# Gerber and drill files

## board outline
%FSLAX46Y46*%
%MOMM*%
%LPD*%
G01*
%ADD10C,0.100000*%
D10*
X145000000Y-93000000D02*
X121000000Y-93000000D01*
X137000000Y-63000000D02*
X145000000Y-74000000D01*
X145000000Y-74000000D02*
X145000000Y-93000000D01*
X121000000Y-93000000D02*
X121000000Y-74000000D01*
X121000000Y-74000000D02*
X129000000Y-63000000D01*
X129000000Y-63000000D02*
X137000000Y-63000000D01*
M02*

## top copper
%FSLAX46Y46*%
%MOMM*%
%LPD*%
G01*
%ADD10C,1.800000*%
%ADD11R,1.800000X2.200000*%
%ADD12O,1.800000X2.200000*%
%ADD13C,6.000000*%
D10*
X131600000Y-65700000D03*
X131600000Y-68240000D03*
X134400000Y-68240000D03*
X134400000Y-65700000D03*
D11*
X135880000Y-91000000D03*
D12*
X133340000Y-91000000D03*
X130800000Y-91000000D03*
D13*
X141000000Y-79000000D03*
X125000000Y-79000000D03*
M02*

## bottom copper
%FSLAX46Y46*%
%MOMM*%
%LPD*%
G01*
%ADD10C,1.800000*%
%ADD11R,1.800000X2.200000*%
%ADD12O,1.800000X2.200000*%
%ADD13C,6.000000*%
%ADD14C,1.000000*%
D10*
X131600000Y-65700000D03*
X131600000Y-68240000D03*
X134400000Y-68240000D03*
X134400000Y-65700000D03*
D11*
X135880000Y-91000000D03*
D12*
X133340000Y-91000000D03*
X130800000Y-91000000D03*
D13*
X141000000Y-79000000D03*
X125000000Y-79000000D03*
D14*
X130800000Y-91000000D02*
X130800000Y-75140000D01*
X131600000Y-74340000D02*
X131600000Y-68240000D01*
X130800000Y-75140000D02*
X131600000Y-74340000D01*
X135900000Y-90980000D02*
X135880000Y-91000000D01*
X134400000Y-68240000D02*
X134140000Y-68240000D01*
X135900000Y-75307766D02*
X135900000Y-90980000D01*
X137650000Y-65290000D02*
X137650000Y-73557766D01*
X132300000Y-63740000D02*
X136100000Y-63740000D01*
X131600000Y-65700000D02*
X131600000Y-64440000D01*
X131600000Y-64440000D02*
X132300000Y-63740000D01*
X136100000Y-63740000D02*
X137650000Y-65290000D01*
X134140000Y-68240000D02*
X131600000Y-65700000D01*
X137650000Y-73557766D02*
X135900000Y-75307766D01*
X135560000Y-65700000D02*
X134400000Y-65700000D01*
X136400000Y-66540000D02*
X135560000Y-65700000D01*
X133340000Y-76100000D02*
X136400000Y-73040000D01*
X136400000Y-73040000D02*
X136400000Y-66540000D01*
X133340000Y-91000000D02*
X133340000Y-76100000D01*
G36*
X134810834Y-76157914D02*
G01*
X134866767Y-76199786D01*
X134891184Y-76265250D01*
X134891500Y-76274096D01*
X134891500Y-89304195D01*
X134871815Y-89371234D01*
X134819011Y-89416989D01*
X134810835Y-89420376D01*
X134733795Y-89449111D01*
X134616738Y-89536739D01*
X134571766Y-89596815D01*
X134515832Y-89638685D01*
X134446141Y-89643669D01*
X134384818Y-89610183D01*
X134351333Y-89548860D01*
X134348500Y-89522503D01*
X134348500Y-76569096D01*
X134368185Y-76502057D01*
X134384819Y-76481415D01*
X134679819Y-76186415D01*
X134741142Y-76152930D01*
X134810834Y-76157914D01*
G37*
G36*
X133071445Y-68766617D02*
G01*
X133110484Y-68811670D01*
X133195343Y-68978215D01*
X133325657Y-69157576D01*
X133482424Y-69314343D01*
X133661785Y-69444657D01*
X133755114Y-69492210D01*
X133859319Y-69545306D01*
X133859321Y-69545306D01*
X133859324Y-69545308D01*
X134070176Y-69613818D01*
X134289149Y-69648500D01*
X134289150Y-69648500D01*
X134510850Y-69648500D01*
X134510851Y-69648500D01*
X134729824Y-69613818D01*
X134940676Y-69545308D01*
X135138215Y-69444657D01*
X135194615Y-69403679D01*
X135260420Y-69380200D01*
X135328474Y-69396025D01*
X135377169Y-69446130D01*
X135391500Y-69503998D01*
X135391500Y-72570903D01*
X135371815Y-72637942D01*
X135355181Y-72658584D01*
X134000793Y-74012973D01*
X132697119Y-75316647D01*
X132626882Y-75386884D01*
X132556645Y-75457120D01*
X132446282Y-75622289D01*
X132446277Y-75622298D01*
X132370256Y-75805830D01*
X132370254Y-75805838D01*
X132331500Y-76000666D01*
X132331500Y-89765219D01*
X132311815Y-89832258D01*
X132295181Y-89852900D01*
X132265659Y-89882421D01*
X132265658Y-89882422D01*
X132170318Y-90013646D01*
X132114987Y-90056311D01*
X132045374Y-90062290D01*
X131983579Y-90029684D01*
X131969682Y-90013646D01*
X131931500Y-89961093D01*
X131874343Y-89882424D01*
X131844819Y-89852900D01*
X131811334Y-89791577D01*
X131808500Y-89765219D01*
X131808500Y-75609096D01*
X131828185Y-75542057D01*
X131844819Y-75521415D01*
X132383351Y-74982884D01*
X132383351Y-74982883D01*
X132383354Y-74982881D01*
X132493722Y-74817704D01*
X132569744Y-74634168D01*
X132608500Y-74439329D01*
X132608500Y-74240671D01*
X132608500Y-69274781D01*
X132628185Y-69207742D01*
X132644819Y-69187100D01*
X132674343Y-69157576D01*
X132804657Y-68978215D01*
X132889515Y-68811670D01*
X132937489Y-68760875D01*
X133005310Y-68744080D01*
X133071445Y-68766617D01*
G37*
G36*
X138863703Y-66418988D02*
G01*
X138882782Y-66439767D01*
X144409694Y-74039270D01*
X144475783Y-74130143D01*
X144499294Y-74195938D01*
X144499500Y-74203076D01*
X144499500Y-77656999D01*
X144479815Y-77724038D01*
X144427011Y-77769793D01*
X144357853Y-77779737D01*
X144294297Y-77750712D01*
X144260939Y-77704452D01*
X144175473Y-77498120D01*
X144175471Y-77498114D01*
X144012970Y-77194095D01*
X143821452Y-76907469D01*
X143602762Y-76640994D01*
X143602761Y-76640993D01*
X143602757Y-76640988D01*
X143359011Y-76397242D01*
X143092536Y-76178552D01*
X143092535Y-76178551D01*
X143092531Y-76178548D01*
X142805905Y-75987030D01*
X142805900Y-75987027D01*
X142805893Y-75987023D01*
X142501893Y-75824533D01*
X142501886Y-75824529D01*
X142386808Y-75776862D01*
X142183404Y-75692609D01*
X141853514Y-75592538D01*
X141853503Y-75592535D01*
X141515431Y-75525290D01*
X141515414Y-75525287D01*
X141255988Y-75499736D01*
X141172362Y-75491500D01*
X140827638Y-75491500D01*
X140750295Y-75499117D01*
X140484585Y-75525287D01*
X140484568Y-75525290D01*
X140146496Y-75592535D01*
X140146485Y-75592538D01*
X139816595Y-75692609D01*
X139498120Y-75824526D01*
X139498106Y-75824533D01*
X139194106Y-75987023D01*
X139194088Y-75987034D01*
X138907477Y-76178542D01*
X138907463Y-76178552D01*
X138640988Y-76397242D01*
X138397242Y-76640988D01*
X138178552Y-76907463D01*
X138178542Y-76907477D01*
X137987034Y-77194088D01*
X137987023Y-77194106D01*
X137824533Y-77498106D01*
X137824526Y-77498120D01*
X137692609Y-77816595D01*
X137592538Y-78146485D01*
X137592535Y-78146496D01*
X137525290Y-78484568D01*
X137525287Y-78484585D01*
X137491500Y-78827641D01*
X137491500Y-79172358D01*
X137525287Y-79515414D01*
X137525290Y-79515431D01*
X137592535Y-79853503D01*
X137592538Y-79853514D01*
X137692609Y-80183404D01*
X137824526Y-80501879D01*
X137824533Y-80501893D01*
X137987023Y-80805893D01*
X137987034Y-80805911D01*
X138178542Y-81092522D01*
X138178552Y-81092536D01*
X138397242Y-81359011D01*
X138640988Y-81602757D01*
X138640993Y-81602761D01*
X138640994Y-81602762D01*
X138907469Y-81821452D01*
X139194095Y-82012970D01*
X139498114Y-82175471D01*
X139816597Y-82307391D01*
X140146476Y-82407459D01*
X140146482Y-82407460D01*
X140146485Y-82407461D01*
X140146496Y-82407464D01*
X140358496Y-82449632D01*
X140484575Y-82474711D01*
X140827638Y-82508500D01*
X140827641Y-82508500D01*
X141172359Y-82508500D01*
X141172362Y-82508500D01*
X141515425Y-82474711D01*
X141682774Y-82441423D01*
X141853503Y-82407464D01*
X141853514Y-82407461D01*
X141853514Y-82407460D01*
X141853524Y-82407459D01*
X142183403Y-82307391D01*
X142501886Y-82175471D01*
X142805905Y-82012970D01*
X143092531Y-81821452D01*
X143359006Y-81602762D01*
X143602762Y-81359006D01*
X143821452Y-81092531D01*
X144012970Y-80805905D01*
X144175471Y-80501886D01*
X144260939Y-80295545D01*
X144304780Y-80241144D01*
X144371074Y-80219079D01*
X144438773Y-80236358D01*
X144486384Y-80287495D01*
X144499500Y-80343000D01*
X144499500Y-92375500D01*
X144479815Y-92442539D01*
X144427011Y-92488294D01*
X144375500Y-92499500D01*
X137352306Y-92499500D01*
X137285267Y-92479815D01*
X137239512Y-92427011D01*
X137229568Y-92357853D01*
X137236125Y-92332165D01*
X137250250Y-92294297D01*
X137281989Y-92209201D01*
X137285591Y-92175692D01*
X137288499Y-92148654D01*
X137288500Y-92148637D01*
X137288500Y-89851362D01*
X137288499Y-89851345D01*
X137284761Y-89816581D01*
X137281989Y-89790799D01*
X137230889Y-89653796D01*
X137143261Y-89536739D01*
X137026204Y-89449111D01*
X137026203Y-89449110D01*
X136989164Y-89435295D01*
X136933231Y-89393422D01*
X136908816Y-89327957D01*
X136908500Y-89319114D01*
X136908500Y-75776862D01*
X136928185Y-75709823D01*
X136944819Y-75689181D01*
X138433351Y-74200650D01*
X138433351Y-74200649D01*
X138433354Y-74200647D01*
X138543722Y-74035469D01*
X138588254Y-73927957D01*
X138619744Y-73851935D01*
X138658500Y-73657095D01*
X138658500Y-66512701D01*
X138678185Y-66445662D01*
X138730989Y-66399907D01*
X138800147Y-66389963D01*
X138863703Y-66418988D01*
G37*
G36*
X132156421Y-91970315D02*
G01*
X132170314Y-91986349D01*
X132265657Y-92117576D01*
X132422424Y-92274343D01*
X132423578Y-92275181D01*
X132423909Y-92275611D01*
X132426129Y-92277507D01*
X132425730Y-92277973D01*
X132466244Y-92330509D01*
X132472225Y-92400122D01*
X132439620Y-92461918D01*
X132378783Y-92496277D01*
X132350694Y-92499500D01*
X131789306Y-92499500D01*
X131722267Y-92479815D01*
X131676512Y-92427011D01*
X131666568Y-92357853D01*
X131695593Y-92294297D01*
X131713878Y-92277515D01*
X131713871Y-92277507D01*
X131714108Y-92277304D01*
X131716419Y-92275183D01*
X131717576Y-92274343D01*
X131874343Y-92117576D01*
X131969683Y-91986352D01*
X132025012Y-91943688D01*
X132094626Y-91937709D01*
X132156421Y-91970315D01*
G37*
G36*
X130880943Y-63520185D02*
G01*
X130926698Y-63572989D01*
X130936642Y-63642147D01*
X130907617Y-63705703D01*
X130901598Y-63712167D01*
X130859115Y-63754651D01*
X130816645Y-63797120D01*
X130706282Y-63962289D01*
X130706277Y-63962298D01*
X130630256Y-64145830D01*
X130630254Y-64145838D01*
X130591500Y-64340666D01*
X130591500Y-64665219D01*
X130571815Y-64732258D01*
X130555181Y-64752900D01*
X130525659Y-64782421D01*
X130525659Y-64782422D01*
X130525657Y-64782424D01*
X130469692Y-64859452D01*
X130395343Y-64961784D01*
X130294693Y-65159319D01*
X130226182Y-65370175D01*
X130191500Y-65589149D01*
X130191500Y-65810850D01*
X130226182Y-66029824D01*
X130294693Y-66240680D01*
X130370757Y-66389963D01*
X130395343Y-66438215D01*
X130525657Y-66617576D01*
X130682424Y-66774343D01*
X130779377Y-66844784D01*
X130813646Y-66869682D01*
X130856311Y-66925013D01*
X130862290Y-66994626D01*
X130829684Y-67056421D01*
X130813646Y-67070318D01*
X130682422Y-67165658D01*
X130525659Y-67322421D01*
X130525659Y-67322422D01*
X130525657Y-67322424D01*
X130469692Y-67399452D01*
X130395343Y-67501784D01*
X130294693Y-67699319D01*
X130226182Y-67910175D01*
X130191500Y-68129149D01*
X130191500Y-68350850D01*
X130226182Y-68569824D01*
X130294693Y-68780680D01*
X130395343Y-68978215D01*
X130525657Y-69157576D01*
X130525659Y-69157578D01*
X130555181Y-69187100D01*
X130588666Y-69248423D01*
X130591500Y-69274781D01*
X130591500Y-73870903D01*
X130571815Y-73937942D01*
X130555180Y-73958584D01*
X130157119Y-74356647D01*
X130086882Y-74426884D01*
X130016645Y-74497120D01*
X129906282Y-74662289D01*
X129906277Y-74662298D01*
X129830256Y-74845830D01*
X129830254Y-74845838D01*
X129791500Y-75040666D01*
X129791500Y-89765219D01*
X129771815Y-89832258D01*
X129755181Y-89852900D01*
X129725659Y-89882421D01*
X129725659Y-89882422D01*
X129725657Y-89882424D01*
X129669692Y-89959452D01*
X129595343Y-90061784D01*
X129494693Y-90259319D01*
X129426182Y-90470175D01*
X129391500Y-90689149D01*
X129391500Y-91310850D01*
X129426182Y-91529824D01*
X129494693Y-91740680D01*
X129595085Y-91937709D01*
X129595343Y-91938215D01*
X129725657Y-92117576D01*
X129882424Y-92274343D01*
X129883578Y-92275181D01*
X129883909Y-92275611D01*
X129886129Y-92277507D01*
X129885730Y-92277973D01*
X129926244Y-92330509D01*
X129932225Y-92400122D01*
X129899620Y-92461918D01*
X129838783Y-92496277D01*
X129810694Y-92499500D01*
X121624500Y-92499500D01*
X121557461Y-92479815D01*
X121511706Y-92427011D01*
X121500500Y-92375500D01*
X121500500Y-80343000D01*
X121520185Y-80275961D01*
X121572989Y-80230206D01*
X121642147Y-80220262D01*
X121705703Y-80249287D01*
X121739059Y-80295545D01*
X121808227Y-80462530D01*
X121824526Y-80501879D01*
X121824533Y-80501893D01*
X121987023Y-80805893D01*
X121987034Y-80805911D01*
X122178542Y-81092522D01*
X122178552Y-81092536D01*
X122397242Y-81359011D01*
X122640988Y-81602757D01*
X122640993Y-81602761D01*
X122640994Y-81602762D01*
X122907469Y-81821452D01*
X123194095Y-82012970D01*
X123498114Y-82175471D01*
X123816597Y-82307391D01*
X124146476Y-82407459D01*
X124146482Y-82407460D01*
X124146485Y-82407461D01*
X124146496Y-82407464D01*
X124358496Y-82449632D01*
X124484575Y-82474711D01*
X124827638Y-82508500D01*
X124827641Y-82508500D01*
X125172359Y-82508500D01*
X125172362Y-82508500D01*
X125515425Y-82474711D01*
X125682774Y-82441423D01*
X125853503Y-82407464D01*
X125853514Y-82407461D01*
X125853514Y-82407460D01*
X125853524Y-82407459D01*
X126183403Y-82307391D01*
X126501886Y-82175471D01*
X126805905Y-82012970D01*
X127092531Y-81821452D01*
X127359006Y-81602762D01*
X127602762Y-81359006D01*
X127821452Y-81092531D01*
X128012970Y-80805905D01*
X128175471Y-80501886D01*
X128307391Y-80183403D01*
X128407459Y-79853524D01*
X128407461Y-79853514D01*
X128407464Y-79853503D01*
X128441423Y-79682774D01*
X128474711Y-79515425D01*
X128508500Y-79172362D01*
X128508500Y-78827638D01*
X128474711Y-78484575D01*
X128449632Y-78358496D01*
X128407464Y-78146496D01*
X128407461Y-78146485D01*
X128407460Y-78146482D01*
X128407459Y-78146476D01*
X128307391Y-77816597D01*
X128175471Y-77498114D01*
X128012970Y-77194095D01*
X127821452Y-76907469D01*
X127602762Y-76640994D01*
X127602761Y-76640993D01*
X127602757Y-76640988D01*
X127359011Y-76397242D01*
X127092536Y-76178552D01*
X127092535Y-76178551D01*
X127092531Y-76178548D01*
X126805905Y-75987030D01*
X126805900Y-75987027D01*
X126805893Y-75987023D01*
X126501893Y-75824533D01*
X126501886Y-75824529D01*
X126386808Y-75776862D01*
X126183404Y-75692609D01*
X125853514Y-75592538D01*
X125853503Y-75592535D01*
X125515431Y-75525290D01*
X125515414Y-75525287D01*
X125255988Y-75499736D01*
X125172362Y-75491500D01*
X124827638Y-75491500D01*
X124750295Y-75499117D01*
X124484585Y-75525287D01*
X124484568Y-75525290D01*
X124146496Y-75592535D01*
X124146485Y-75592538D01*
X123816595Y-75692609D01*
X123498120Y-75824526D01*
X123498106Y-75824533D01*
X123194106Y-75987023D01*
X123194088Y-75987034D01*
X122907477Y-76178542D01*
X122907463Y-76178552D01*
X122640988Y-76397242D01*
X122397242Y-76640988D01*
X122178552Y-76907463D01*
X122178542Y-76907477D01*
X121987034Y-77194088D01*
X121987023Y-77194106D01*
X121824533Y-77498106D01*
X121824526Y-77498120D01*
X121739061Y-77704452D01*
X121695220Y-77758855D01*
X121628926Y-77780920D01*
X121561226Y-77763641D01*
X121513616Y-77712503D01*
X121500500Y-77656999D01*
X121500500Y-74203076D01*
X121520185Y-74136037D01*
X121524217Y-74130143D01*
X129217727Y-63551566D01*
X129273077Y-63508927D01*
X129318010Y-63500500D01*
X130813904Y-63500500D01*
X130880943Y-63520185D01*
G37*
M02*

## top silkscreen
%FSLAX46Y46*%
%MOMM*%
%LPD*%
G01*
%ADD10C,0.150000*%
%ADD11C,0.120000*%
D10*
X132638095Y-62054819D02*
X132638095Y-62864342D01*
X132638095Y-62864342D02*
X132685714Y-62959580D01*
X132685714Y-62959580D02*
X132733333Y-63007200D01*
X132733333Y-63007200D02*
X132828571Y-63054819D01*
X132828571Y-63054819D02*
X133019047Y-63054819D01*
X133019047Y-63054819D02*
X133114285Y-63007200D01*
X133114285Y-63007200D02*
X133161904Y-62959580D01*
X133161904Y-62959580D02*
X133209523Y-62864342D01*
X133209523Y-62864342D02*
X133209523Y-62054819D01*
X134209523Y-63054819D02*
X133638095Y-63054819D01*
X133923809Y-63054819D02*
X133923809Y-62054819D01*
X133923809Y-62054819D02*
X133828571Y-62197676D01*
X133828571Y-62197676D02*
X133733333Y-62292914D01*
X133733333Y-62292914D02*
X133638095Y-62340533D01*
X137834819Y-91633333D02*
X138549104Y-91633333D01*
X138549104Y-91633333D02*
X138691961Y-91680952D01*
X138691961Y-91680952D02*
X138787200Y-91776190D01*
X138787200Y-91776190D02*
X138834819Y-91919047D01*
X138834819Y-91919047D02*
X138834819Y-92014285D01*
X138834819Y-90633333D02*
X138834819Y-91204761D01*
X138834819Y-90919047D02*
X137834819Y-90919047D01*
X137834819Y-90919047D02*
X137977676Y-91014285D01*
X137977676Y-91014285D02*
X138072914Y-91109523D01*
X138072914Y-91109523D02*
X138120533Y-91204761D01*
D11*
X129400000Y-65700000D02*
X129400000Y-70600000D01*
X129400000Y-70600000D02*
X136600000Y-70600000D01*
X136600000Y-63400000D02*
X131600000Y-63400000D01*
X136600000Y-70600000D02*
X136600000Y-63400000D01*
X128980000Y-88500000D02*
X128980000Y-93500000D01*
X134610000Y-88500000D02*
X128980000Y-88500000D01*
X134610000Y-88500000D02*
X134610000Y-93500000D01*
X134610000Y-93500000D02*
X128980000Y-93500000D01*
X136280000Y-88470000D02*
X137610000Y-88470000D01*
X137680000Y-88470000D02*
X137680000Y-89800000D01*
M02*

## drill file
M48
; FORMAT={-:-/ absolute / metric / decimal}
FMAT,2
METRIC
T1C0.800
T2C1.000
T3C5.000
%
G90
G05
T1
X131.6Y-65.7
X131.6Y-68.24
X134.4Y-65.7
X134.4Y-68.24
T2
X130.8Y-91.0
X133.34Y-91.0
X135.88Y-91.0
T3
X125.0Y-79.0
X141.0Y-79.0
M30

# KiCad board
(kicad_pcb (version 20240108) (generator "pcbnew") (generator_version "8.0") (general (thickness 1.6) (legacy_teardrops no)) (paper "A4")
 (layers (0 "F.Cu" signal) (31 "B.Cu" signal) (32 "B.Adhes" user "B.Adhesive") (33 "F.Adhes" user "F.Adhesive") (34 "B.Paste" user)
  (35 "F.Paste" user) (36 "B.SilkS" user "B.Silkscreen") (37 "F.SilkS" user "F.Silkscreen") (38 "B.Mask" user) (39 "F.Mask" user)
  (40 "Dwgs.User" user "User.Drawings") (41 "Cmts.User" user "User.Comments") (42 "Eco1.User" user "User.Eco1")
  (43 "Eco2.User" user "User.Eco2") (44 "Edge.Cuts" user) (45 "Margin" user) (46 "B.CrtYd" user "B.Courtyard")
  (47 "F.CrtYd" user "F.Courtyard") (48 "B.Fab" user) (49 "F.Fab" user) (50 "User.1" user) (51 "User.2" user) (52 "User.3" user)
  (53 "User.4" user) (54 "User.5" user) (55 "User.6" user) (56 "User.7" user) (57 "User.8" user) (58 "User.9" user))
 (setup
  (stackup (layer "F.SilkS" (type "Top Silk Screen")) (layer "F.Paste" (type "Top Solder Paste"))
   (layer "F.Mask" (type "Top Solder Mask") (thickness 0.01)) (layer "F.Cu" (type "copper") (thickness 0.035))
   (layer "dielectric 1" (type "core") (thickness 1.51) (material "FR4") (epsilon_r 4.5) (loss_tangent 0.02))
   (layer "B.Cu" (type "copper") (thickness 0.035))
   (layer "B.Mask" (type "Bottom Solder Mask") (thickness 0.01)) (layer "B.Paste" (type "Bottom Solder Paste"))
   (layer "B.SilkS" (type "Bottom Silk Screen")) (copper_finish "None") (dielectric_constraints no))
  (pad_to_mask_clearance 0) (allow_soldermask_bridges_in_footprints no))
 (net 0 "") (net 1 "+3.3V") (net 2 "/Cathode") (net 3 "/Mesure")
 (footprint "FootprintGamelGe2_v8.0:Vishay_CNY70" (layer "F.Cu") (at 131.6 65.7)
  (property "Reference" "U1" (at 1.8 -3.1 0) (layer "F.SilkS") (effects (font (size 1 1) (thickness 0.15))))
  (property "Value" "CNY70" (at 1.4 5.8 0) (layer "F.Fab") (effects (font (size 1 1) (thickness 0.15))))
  (fp_line (start -2.2 0) (end -2.2 4.9) (stroke (width 0.12) (type solid)) (layer "F.SilkS"))
  (fp_line (start -2.2 4.9) (end 5 4.9) (stroke (width 0.12) (type solid)) (layer "F.SilkS"))
  (fp_line (start 5 -2.3) (end 0 -2.3) (stroke (width 0.12) (type solid)) (layer "F.SilkS"))
  (fp_line (start 5 4.9) (end 5 -2.3) (stroke (width 0.12) (type solid)) (layer "F.SilkS"))
  (pad "1" thru_hole circle (at 0 0) (size 1.8 1.8) (drill 0.8) (layers "*.Cu" "*.Mask") (remove_unused_layers no) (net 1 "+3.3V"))
  (pad "2" thru_hole circle (at 0 2.54) (size 1.8 1.8) (drill 0.8) (layers "*.Cu" "*.Mask") (remove_unused_layers no) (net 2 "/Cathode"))
  (pad "3" thru_hole circle (at 2.8 2.54) (size 1.8 1.8) (drill 0.8) (layers "*.Cu" "*.Mask") (remove_unused_layers no) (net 1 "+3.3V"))
  (pad "4" thru_hole circle (at 2.8 0) (size 1.8 1.8) (drill 0.8) (layers "*.Cu" "*.Mask") (remove_unused_layers no) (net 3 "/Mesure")))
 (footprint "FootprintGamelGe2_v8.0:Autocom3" (layer "F.Cu") (at 135.88 91 -90)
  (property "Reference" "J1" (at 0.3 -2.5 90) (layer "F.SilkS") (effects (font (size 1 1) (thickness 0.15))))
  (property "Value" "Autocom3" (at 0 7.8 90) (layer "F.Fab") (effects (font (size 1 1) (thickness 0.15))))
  (fp_line (start -2.5 6.9) (end 2.5 6.9) (stroke (width 0.12) (type solid)) (layer "F.SilkS"))
  (fp_line (start -2.5 1.27) (end -2.5 6.9) (stroke (width 0.12) (type solid)) (layer "F.SilkS"))
  (fp_line (start -2.5 1.27) (end 2.5 1.27) (stroke (width 0.12) (type solid)) (layer "F.SilkS"))
  (fp_line (start 2.5 1.27) (end 2.5 6.9) (stroke (width 0.12) (type solid)) (layer "F.SilkS"))
  (fp_line (start -2.53 -0.4) (end -2.53 -1.73) (stroke (width 0.12) (type solid)) (layer "F.SilkS"))
  (fp_line (start -2.53 -1.8) (end -1.2 -1.8) (stroke (width 0.12) (type solid)) (layer "F.SilkS"))
  (pad "1" thru_hole rect (at 0 0 270) (size 2.2 1.8) (drill 1) (layers "*.Cu" "*.Mask") (remove_unused_layers no) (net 1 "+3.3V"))
  (pad "2" thru_hole oval (at 0 2.54 270) (size 2.2 1.8) (drill 1) (layers "*.Cu" "*.Mask") (remove_unused_layers no) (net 3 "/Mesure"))
  (pad "3" thru_hole oval (at 0 5.08 270) (size 2.2 1.8) (drill 1) (layers "*.Cu" "*.Mask") (remove_unused_layers no) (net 2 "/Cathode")))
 (gr_line (start 145 93) (end 121 93) (stroke (width 0.1) (type default)) (layer "Edge.Cuts"))
 (gr_line (start 137 63) (end 145 74) (stroke (width 0.1) (type default)) (layer "Edge.Cuts"))
 (gr_line (start 145 74) (end 145 93) (stroke (width 0.1) (type default)) (layer "Edge.Cuts"))
 (gr_line (start 121 93) (end 121 74) (stroke (width 0.1) (type default)) (layer "Edge.Cuts"))
 (gr_line (start 121 74) (end 129 63) (stroke (width 0.1) (type default)) (layer "Edge.Cuts"))
 (gr_line (start 129 63) (end 137 63) (stroke (width 0.1) (type default)) (layer "Edge.Cuts"))
 (via (at 141 79) (size 6) (drill 5) (layers "F.Cu" "B.Cu") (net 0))
 (via (at 125 79) (size 6) (drill 5) (layers "F.Cu" "B.Cu") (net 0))
 (segment (start 130.8 91) (end 130.8 75.14) (width 1) (layer "B.Cu") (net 2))
 (segment (start 131.6 74.34) (end 131.6 68.24) (width 1) (layer "B.Cu") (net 2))
 (segment (start 130.8 75.14) (end 131.6 74.34) (width 1) (layer "B.Cu") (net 2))
 (segment (start 135.9 90.98) (end 135.88 91) (width 1) (layer "B.Cu") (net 1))
 (segment (start 134.4 68.24) (end 134.14 68.24) (width 1) (layer "B.Cu") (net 1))
 (segment (start 135.9 75.307766) (end 135.9 90.98) (width 1) (layer "B.Cu") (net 1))
 (segment (start 137.65 65.29) (end 137.65 73.557766) (width 1) (layer "B.Cu") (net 1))
 (segment (start 132.3 63.74) (end 136.1 63.74) (width 1) (layer "B.Cu") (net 1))
 (segment (start 131.6 65.7) (end 131.6 64.44) (width 1) (layer "B.Cu") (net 1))
 (segment (start 131.6 64.44) (end 132.3 63.74) (width 1) (layer "B.Cu") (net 1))
 (segment (start 136.1 63.74) (end 137.65 65.29) (width 1) (layer "B.Cu") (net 1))
 (segment (start 134.14 68.24) (end 131.6 65.7) (width 1) (layer "B.Cu") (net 1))
 (segment (start 137.65 73.557766) (end 135.9 75.307766) (width 1) (layer "B.Cu") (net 1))
 (segment (start 135.56 65.7) (end 134.4 65.7) (width 1) (layer "B.Cu") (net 3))
 (segment (start 136.4 66.54) (end 135.56 65.7) (width 1) (layer "B.Cu") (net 3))
 (segment (start 133.34 76.1) (end 136.4 73.04) (width 1) (layer "B.Cu") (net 3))
 (segment (start 136.4 73.04) (end 136.4 66.54) (width 1) (layer "B.Cu") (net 3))
 (segment (start 133.34 91) (end 133.34 76.1) (width 1) (layer "B.Cu") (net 3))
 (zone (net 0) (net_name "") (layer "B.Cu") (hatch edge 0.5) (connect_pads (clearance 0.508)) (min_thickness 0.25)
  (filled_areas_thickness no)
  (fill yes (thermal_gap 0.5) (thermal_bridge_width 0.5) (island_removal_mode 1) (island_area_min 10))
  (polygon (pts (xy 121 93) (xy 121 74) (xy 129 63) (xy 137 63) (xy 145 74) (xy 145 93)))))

